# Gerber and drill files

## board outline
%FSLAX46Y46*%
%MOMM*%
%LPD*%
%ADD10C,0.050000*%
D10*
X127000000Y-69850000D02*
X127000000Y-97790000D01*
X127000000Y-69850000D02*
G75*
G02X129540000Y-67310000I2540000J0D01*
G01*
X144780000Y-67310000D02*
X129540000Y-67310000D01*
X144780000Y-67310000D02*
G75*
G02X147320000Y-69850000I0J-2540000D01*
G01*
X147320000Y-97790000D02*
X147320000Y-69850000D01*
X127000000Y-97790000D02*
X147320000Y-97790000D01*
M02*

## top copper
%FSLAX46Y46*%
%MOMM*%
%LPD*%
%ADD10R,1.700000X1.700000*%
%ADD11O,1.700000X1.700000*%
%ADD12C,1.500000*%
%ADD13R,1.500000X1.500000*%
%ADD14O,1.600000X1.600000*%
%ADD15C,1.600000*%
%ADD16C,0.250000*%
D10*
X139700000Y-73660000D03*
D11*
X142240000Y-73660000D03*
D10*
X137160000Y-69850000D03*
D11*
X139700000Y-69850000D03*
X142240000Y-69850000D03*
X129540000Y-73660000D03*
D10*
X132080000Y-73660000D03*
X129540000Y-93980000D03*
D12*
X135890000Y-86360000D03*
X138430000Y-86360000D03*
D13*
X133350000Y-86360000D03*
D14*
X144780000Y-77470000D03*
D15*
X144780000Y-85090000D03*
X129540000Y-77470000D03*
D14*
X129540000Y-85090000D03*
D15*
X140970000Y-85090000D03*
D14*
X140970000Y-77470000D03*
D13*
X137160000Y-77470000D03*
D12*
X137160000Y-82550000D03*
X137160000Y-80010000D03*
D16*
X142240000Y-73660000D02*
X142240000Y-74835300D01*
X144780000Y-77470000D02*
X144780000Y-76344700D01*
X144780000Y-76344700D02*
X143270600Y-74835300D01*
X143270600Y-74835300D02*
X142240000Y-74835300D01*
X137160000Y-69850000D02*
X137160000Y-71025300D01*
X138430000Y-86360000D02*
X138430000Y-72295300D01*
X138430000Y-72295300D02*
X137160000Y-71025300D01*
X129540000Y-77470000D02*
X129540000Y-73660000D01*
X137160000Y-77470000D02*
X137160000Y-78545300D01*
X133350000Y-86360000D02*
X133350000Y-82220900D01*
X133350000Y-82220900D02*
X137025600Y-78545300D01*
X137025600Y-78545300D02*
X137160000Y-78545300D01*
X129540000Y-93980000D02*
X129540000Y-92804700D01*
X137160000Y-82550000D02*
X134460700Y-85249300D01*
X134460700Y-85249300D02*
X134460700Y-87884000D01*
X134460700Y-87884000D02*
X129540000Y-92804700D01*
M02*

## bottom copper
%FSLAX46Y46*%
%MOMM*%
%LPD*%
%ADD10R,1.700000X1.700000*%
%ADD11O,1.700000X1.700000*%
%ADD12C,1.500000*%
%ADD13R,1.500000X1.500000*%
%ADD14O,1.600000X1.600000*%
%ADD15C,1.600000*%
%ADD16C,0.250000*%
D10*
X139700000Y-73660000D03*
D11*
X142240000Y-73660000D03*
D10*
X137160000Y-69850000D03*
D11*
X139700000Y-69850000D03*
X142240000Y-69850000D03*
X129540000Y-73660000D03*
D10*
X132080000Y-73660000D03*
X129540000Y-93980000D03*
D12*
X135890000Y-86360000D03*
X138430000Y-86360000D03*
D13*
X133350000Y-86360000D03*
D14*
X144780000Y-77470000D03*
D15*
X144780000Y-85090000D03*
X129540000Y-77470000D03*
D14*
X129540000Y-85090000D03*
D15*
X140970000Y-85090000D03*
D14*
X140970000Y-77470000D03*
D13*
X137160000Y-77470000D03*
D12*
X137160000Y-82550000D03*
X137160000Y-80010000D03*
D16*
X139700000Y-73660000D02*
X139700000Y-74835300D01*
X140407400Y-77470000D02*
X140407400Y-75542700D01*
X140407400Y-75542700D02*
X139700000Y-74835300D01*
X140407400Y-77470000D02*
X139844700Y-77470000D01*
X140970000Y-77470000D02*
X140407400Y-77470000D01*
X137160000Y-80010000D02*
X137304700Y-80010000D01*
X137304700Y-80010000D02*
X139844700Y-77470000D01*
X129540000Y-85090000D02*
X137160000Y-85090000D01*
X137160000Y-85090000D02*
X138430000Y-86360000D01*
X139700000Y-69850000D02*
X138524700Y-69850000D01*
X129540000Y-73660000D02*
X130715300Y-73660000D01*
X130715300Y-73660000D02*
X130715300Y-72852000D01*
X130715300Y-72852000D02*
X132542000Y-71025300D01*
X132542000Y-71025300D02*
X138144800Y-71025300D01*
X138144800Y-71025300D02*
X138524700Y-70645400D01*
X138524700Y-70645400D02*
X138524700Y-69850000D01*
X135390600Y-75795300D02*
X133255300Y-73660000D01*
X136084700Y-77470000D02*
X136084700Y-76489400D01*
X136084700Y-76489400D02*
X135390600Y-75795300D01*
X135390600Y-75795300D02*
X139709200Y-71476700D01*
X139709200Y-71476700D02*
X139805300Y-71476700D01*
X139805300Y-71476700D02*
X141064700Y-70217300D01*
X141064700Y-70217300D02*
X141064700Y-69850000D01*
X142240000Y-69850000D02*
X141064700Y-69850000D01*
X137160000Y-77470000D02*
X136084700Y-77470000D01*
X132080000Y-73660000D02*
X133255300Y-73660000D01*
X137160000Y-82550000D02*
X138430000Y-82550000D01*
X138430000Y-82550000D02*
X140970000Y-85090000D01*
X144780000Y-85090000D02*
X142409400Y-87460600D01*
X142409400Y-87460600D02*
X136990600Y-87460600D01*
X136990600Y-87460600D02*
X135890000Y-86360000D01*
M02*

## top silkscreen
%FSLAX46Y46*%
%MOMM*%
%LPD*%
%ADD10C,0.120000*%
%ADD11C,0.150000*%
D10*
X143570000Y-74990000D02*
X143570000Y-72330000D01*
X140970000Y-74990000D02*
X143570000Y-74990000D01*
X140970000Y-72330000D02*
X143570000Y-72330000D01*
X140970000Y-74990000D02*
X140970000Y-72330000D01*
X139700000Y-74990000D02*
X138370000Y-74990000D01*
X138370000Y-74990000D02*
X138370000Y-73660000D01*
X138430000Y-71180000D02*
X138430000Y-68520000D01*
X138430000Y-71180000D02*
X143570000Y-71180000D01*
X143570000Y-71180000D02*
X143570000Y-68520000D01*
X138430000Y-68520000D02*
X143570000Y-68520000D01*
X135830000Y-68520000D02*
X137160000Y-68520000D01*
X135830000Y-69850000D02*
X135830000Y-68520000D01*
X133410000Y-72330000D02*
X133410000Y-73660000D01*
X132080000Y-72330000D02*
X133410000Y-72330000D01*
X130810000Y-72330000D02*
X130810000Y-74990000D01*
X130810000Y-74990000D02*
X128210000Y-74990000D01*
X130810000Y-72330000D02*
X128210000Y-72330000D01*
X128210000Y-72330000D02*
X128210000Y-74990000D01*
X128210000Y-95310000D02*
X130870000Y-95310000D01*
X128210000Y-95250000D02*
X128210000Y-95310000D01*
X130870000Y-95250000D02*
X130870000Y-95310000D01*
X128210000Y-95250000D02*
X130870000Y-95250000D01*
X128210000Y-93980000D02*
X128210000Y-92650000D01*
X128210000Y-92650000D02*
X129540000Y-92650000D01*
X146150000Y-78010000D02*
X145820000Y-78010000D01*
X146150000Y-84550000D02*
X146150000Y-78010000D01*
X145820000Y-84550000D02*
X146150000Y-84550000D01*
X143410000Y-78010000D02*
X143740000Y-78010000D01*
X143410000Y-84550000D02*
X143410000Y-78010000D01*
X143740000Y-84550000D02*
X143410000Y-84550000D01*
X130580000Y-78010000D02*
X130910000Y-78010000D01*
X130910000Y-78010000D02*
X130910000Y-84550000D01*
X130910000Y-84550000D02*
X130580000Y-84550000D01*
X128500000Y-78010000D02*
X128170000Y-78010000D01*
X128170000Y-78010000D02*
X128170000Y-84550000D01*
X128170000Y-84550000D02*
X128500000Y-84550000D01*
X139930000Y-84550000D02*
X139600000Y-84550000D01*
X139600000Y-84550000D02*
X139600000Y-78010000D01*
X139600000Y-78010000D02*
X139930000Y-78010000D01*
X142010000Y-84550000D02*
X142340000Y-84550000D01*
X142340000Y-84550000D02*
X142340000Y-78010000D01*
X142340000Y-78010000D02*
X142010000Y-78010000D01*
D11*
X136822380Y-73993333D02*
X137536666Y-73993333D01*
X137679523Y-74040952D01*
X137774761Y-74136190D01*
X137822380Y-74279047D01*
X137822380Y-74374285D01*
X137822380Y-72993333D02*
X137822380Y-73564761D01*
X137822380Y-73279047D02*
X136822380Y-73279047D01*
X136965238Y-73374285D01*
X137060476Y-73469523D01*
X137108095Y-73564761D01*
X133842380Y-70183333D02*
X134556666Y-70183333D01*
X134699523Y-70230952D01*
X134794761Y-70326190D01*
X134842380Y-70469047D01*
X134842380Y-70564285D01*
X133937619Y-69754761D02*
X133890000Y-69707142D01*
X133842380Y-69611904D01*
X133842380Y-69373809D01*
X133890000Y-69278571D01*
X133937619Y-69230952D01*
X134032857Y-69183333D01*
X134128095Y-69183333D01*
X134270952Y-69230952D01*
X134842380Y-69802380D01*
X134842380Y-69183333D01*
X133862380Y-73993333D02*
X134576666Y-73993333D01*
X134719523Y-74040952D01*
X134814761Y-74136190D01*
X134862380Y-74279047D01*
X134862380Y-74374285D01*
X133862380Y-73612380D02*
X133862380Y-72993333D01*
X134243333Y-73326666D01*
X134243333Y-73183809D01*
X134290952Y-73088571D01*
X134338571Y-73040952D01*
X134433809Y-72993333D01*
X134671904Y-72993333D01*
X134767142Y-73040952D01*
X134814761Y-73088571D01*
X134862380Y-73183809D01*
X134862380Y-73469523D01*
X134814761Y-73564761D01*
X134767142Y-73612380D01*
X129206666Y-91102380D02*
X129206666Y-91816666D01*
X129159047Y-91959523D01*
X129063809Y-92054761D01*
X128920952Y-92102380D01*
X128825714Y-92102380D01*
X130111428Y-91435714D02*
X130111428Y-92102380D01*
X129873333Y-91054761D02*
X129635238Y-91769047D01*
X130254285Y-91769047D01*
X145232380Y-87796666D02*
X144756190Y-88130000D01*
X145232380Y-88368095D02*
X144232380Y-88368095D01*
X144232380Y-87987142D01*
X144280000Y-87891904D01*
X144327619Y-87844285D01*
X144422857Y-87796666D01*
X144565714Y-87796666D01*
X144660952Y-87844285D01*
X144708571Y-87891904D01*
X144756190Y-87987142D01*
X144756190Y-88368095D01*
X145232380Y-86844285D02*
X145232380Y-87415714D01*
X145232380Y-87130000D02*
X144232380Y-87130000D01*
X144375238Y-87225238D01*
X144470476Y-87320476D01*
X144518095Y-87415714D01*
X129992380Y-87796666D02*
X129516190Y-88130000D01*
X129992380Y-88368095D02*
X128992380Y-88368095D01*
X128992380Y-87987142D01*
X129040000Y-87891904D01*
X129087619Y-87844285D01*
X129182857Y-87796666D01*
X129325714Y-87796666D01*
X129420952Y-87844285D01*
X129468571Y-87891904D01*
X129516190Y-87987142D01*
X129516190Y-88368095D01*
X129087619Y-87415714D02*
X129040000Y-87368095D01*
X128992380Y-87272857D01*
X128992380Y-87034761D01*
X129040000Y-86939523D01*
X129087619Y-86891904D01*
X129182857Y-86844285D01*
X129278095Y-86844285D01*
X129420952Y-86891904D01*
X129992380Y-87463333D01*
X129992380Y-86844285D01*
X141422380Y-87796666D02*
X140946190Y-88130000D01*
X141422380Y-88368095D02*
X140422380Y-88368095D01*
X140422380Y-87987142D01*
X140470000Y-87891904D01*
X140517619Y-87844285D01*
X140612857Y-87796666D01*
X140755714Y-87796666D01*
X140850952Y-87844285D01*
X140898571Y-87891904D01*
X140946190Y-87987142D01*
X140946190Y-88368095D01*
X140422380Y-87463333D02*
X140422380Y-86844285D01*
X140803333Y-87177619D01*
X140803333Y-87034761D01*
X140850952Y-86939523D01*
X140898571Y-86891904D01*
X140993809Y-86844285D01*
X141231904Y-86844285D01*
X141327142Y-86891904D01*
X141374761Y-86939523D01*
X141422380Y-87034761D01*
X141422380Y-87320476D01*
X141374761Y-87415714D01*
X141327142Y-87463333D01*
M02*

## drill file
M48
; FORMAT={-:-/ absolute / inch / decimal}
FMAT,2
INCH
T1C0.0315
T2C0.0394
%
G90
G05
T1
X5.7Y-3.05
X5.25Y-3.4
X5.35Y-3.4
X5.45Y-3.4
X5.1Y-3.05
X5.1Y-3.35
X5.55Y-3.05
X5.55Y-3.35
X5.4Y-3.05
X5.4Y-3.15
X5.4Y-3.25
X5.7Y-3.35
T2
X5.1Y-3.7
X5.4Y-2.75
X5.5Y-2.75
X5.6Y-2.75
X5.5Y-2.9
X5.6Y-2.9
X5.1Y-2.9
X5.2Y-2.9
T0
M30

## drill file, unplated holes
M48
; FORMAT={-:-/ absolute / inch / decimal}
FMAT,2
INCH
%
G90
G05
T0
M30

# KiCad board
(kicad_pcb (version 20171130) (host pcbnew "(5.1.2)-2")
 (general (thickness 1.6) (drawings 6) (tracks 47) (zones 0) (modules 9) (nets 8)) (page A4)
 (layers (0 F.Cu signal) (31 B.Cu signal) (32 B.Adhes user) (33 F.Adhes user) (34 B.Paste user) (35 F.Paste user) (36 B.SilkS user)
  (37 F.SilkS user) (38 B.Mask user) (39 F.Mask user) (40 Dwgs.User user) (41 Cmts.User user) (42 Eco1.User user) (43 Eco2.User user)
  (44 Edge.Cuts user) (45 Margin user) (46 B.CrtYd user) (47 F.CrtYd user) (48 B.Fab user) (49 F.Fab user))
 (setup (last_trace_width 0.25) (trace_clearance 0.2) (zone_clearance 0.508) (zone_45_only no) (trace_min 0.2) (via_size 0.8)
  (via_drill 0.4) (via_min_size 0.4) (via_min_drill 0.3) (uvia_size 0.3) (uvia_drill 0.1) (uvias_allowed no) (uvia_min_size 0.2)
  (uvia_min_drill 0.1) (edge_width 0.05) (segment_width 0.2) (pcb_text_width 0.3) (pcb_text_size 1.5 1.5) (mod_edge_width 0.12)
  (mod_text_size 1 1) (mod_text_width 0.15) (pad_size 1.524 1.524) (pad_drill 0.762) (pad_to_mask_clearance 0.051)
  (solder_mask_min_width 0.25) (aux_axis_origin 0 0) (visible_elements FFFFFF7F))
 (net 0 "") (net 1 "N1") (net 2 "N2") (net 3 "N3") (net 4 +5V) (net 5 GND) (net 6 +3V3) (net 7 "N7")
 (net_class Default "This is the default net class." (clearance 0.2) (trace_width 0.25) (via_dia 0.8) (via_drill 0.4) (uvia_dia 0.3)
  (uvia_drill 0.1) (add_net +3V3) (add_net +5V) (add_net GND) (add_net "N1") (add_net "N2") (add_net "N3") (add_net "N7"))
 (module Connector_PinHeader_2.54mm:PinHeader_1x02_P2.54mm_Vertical (layer F.Cu) (at 139.7 73.66 90)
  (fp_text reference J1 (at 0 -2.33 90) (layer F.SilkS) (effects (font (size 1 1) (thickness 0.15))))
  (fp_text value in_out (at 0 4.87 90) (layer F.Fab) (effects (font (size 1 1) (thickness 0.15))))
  (fp_line (start -1.33 3.87) (end 1.33 3.87) (layer F.SilkS) (width 0.12))
  (fp_line (start -1.33 1.27) (end -1.33 3.87) (layer F.SilkS) (width 0.12))
  (fp_line (start 1.33 1.27) (end 1.33 3.87) (layer F.SilkS) (width 0.12))
  (fp_line (start -1.33 1.27) (end 1.33 1.27) (layer F.SilkS) (width 0.12))
  (fp_line (start -1.33 0) (end -1.33 -1.33) (layer F.SilkS) (width 0.12))
  (fp_line (start -1.33 -1.33) (end 0 -1.33) (layer F.SilkS) (width 0.12))
  (pad 1 thru_hole rect (at 0 0 90) (size 1.7 1.7) (drill 1) (layers *.Cu *.Mask) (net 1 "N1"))
  (pad 2 thru_hole oval (at 0 2.54 90) (size 1.7 1.7) (drill 1) (layers *.Cu *.Mask) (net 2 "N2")))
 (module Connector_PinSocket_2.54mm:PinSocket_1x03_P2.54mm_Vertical (layer F.Cu) (at 137.16 69.85 90)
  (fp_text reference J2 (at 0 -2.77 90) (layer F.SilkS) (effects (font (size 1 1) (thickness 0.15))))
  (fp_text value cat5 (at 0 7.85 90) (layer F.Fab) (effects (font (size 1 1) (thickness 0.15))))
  (fp_line (start -1.33 1.27) (end 1.33 1.27) (layer F.SilkS) (width 0.12))
  (fp_line (start -1.33 1.27) (end -1.33 6.41) (layer F.SilkS) (width 0.12))
  (fp_line (start -1.33 6.41) (end 1.33 6.41) (layer F.SilkS) (width 0.12))
  (fp_line (start 1.33 1.27) (end 1.33 6.41) (layer F.SilkS) (width 0.12))
  (fp_line (start 1.33 -1.33) (end 1.33 0) (layer F.SilkS) (width 0.12))
  (fp_line (start 0 -1.33) (end 1.33 -1.33) (layer F.SilkS) (width 0.12))
  (pad 1 thru_hole rect (at 0 0 90) (size 1.7 1.7) (drill 1) (layers *.Cu *.Mask) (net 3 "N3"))
  (pad 2 thru_hole oval (at 0 2.54 90) (size 1.7 1.7) (drill 1) (layers *.Cu *.Mask) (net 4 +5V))
  (pad 3 thru_hole oval (at 0 5.08 90) (size 1.7 1.7) (drill 1) (layers *.Cu *.Mask) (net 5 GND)))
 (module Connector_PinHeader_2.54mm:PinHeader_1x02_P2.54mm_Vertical (layer F.Cu) (at 132.08 73.66 270)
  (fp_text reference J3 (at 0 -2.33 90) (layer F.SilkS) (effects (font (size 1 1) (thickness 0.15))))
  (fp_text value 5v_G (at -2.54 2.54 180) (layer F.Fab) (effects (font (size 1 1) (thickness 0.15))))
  (fp_line (start -1.33 -1.33) (end 0 -1.33) (layer F.SilkS) (width 0.12))
  (fp_line (start -1.33 0) (end -1.33 -1.33) (layer F.SilkS) (width 0.12))
  (fp_line (start -1.33 1.27) (end 1.33 1.27) (layer F.SilkS) (width 0.12))
  (fp_line (start 1.33 1.27) (end 1.33 3.87) (layer F.SilkS) (width 0.12))
  (fp_line (start -1.33 1.27) (end -1.33 3.87) (layer F.SilkS) (width 0.12))
  (fp_line (start -1.33 3.87) (end 1.33 3.87) (layer F.SilkS) (width 0.12))
  (pad 2 thru_hole oval (at 0 2.54 270) (size 1.7 1.7) (drill 1) (layers *.Cu *.Mask) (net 4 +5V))
  (pad 1 thru_hole rect (at 0 0 270) (size 1.7 1.7) (drill 1) (layers *.Cu *.Mask) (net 5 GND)))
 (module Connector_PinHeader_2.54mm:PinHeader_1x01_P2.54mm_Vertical (layer F.Cu) (at 129.54 93.98)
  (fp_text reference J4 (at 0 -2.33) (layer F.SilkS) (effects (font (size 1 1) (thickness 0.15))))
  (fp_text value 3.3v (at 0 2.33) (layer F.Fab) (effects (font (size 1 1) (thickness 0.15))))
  (fp_line (start -1.33 1.33) (end 1.33 1.33) (layer F.SilkS) (width 0.12))
  (fp_line (start -1.33 1.27) (end -1.33 1.33) (layer F.SilkS) (width 0.12))
  (fp_line (start 1.33 1.27) (end 1.33 1.33) (layer F.SilkS) (width 0.12))
  (fp_line (start -1.33 1.27) (end 1.33 1.27) (layer F.SilkS) (width 0.12))
  (fp_line (start -1.33 0) (end -1.33 -1.33) (layer F.SilkS) (width 0.12))
  (fp_line (start -1.33 -1.33) (end 0 -1.33) (layer F.SilkS) (width 0.12))
  (pad 1 thru_hole rect (at 0 0) (size 1.7 1.7) (drill 1) (layers *.Cu *.Mask) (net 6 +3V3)))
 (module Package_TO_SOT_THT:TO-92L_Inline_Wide (layer B.Cu) (at 133.35 86.36)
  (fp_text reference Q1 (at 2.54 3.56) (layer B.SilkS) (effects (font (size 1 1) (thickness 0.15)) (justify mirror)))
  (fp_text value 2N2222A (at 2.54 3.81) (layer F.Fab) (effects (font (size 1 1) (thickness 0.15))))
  (pad 2 thru_hole circle (at 2.54 0 270) (size 1.5 1.5) (drill 0.8) (layers *.Cu *.Mask) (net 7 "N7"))
  (pad 3 thru_hole circle (at 5.08 0 270) (size 1.5 1.5) (drill 0.8) (layers *.Cu *.Mask) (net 3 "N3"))
  (pad 1 thru_hole rect (at 0 0 270) (size 1.5 1.5) (drill 0.8) (layers *.Cu *.Mask) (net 5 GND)))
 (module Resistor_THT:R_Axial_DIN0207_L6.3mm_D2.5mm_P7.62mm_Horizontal (layer F.Cu) (at 144.78 85.09 90)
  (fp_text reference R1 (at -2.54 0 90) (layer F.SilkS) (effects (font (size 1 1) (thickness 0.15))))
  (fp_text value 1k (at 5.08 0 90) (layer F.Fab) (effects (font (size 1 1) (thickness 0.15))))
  (fp_line (start 7.08 1.37) (end 7.08 1.04) (layer F.SilkS) (width 0.12))
  (fp_line (start 0.54 1.37) (end 7.08 1.37) (layer F.SilkS) (width 0.12))
  (fp_line (start 0.54 1.04) (end 0.54 1.37) (layer F.SilkS) (width 0.12))
  (fp_line (start 7.08 -1.37) (end 7.08 -1.04) (layer F.SilkS) (width 0.12))
  (fp_line (start 0.54 -1.37) (end 7.08 -1.37) (layer F.SilkS) (width 0.12))
  (fp_line (start 0.54 -1.04) (end 0.54 -1.37) (layer F.SilkS) (width 0.12))
  (pad 2 thru_hole oval (at 7.62 0 90) (size 1.6 1.6) (drill 0.8) (layers *.Cu *.Mask) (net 2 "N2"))
  (pad 1 thru_hole circle (at 0 0 90) (size 1.6 1.6) (drill 0.8) (layers *.Cu *.Mask) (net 7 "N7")))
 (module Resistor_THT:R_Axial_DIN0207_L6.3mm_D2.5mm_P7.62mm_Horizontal (layer F.Cu) (at 129.54 77.47 270)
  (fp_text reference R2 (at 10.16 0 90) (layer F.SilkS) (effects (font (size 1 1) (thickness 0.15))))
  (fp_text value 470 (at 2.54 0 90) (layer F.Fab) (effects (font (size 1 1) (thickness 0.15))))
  (fp_line (start 0.54 -1.04) (end 0.54 -1.37) (layer F.SilkS) (width 0.12))
  (fp_line (start 0.54 -1.37) (end 7.08 -1.37) (layer F.SilkS) (width 0.12))
  (fp_line (start 7.08 -1.37) (end 7.08 -1.04) (layer F.SilkS) (width 0.12))
  (fp_line (start 0.54 1.04) (end 0.54 1.37) (layer F.SilkS) (width 0.12))
  (fp_line (start 0.54 1.37) (end 7.08 1.37) (layer F.SilkS) (width 0.12))
  (fp_line (start 7.08 1.37) (end 7.08 1.04) (layer F.SilkS) (width 0.12))
  (pad 1 thru_hole circle (at 0 0 270) (size 1.6 1.6) (drill 0.8) (layers *.Cu *.Mask) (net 4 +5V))
  (pad 2 thru_hole oval (at 7.62 0 270) (size 1.6 1.6) (drill 0.8) (layers *.Cu *.Mask) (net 3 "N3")))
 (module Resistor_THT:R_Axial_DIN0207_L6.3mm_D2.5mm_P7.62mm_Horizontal (layer F.Cu) (at 140.97 85.09 90)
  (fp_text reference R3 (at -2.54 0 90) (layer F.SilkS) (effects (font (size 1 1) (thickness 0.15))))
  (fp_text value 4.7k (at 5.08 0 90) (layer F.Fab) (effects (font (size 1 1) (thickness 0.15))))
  (fp_line (start 0.54 -1.04) (end 0.54 -1.37) (layer F.SilkS) (width 0.12))
  (fp_line (start 0.54 -1.37) (end 7.08 -1.37) (layer F.SilkS) (width 0.12))
  (fp_line (start 7.08 -1.37) (end 7.08 -1.04) (layer F.SilkS) (width 0.12))
  (fp_line (start 0.54 1.04) (end 0.54 1.37) (layer F.SilkS) (width 0.12))
  (fp_line (start 0.54 1.37) (end 7.08 1.37) (layer F.SilkS) (width 0.12))
  (fp_line (start 7.08 1.37) (end 7.08 1.04) (layer F.SilkS) (width 0.12))
  (pad 1 thru_hole circle (at 0 0 90) (size 1.6 1.6) (drill 0.8) (layers *.Cu *.Mask) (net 6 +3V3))
  (pad 2 thru_hole oval (at 7.62 0 90) (size 1.6 1.6) (drill 0.8) (layers *.Cu *.Mask) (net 1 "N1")))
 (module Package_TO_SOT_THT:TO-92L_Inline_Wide (layer B.Cu) (at 137.16 77.47 270)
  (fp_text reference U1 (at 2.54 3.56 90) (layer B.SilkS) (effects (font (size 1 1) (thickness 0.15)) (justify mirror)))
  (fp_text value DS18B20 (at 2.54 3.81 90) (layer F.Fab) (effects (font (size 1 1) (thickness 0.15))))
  (pad 1 thru_hole rect (at 0 0 180) (size 1.5 1.5) (drill 0.8) (layers *.Cu *.Mask) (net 5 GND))
  (pad 3 thru_hole circle (at 5.08 0 180) (size 1.5 1.5) (drill 0.8) (layers *.Cu *.Mask) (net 6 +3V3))
  (pad 2 thru_hole circle (at 2.54 0 180) (size 1.5 1.5) (drill 0.8) (layers *.Cu *.Mask) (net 1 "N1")))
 (gr_line (start 127 69.85) (end 127 97.79) (layer Edge.Cuts) (width 0.05))
 (gr_arc (start 129.54 69.85) (end 129.54 67.31) (angle -90) (layer Edge.Cuts) (width 0.05))
 (gr_line (start 144.78 67.31) (end 129.54 67.31) (layer Edge.Cuts) (width 0.05))
 (gr_arc (start 144.78 69.85) (end 147.32 69.85) (angle -90) (layer Edge.Cuts) (width 0.05))
 (gr_line (start 147.32 97.79) (end 147.32 69.85) (layer Edge.Cuts) (width 0.05))
 (gr_line (start 127 97.79) (end 147.32 97.79) (layer Edge.Cuts) (width 0.05))
 (segment (start 139.7 73.66) (end 139.7 74.8353) (width 0.25) (layer B.Cu) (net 1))
 (segment (start 140.4074 77.47) (end 140.4074 75.5427) (width 0.25) (layer B.Cu) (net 1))
 (segment (start 140.4074 75.5427) (end 139.7 74.8353) (width 0.25) (layer B.Cu) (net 1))
 (segment (start 140.4074 77.47) (end 139.8447 77.47) (width 0.25) (layer B.Cu) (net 1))
 (segment (start 140.97 77.47) (end 140.4074 77.47) (width 0.25) (layer B.Cu) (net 1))
 (segment (start 137.16 80.01) (end 137.3047 80.01) (width 0.25) (layer B.Cu) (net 1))
 (segment (start 137.3047 80.01) (end 139.8447 77.47) (width 0.25) (layer B.Cu) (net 1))
 (segment (start 142.24 73.66) (end 142.24 74.8353) (width 0.25) (layer F.Cu) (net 2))
 (segment (start 144.78 77.47) (end 144.78 76.3447) (width 0.25) (layer F.Cu) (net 2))
 (segment (start 144.78 76.3447) (end 143.2706 74.8353) (width 0.25) (layer F.Cu) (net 2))
 (segment (start 143.2706 74.8353) (end 142.24 74.8353) (width 0.25) (layer F.Cu) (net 2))
 (segment (start 137.16 69.85) (end 137.16 71.0253) (width 0.25) (layer F.Cu) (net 3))
 (segment (start 138.43 86.36) (end 138.43 72.2953) (width 0.25) (layer F.Cu) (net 3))
 (segment (start 138.43 72.2953) (end 137.16 71.0253) (width 0.25) (layer F.Cu) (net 3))
 (segment (start 129.54 85.09) (end 137.16 85.09) (width 0.25) (layer B.Cu) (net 3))
 (segment (start 137.16 85.09) (end 138.43 86.36) (width 0.25) (layer B.Cu) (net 3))
 (segment (start 139.7 69.85) (end 138.5247 69.85) (width 0.25) (layer B.Cu) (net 4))
 (segment (start 129.54 73.66) (end 130.7153 73.66) (width 0.25) (layer B.Cu) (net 4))
 (segment (start 130.7153 73.66) (end 130.7153 72.852) (width 0.25) (layer B.Cu) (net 4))
 (segment (start 130.7153 72.852) (end 132.542 71.0253) (width 0.25) (layer B.Cu) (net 4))
 (segment (start 132.542 71.0253) (end 138.1448 71.0253) (width 0.25) (layer B.Cu) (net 4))
 (segment (start 138.1448 71.0253) (end 138.5247 70.6454) (width 0.25) (layer B.Cu) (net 4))
 (segment (start 138.5247 70.6454) (end 138.5247 69.85) (width 0.25) (layer B.Cu) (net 4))
 (segment (start 129.54 77.47) (end 129.54 73.66) (width 0.25) (layer F.Cu) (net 4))
 (segment (start 135.3906 75.7953) (end 133.2553 73.66) (width 0.25) (layer B.Cu) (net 5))
 (segment (start 136.0847 77.47) (end 136.0847 76.4894) (width 0.25) (layer B.Cu) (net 5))
 (segment (start 136.0847 76.4894) (end 135.3906 75.7953) (width 0.25) (layer B.Cu) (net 5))
 (segment (start 135.3906 75.7953) (end 139.7092 71.4767) (width 0.25) (layer B.Cu) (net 5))
 (segment (start 139.7092 71.4767) (end 139.8053 71.4767) (width 0.25) (layer B.Cu) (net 5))
 (segment (start 139.8053 71.4767) (end 141.0647 70.2173) (width 0.25) (layer B.Cu) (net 5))
 (segment (start 141.0647 70.2173) (end 141.0647 69.85) (width 0.25) (layer B.Cu) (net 5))
 (segment (start 142.24 69.85) (end 141.0647 69.85) (width 0.25) (layer B.Cu) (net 5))
 (segment (start 137.16 77.47) (end 136.0847 77.47) (width 0.25) (layer B.Cu) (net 5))
 (segment (start 132.08 73.66) (end 133.2553 73.66) (width 0.25) (layer B.Cu) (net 5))
 (segment (start 137.16 77.47) (end 137.16 78.5453) (width 0.25) (layer F.Cu) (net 5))
 (segment (start 133.35 86.36) (end 133.35 82.2209) (width 0.25) (layer F.Cu) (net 5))
 (segment (start 133.35 82.2209) (end 137.0256 78.5453) (width 0.25) (layer F.Cu) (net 5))
 (segment (start 137.0256 78.5453) (end 137.16 78.5453) (width 0.25) (layer F.Cu) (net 5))
 (segment (start 129.54 93.98) (end 129.54 92.8047) (width 0.25) (layer F.Cu) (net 6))
 (segment (start 137.16 82.55) (end 134.4607 85.2493) (width 0.25) (layer F.Cu) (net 6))
 (segment (start 134.4607 85.2493) (end 134.4607 87.884) (width 0.25) (layer F.Cu) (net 6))
 (segment (start 134.4607 87.884) (end 129.54 92.8047) (width 0.25) (layer F.Cu) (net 6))
 (segment (start 137.16 82.55) (end 138.43 82.55) (width 0.25) (layer B.Cu) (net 6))
 (segment (start 138.43 82.55) (end 140.97 85.09) (width 0.25) (layer B.Cu) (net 6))
 (segment (start 144.78 85.09) (end 142.4094 87.4606) (width 0.25) (layer B.Cu) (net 7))
 (segment (start 142.4094 87.4606) (end 136.9906 87.4606) (width 0.25) (layer B.Cu) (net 7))
 (segment (start 136.9906 87.4606) (end 135.89 86.36) (width 0.25) (layer B.Cu) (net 7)))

